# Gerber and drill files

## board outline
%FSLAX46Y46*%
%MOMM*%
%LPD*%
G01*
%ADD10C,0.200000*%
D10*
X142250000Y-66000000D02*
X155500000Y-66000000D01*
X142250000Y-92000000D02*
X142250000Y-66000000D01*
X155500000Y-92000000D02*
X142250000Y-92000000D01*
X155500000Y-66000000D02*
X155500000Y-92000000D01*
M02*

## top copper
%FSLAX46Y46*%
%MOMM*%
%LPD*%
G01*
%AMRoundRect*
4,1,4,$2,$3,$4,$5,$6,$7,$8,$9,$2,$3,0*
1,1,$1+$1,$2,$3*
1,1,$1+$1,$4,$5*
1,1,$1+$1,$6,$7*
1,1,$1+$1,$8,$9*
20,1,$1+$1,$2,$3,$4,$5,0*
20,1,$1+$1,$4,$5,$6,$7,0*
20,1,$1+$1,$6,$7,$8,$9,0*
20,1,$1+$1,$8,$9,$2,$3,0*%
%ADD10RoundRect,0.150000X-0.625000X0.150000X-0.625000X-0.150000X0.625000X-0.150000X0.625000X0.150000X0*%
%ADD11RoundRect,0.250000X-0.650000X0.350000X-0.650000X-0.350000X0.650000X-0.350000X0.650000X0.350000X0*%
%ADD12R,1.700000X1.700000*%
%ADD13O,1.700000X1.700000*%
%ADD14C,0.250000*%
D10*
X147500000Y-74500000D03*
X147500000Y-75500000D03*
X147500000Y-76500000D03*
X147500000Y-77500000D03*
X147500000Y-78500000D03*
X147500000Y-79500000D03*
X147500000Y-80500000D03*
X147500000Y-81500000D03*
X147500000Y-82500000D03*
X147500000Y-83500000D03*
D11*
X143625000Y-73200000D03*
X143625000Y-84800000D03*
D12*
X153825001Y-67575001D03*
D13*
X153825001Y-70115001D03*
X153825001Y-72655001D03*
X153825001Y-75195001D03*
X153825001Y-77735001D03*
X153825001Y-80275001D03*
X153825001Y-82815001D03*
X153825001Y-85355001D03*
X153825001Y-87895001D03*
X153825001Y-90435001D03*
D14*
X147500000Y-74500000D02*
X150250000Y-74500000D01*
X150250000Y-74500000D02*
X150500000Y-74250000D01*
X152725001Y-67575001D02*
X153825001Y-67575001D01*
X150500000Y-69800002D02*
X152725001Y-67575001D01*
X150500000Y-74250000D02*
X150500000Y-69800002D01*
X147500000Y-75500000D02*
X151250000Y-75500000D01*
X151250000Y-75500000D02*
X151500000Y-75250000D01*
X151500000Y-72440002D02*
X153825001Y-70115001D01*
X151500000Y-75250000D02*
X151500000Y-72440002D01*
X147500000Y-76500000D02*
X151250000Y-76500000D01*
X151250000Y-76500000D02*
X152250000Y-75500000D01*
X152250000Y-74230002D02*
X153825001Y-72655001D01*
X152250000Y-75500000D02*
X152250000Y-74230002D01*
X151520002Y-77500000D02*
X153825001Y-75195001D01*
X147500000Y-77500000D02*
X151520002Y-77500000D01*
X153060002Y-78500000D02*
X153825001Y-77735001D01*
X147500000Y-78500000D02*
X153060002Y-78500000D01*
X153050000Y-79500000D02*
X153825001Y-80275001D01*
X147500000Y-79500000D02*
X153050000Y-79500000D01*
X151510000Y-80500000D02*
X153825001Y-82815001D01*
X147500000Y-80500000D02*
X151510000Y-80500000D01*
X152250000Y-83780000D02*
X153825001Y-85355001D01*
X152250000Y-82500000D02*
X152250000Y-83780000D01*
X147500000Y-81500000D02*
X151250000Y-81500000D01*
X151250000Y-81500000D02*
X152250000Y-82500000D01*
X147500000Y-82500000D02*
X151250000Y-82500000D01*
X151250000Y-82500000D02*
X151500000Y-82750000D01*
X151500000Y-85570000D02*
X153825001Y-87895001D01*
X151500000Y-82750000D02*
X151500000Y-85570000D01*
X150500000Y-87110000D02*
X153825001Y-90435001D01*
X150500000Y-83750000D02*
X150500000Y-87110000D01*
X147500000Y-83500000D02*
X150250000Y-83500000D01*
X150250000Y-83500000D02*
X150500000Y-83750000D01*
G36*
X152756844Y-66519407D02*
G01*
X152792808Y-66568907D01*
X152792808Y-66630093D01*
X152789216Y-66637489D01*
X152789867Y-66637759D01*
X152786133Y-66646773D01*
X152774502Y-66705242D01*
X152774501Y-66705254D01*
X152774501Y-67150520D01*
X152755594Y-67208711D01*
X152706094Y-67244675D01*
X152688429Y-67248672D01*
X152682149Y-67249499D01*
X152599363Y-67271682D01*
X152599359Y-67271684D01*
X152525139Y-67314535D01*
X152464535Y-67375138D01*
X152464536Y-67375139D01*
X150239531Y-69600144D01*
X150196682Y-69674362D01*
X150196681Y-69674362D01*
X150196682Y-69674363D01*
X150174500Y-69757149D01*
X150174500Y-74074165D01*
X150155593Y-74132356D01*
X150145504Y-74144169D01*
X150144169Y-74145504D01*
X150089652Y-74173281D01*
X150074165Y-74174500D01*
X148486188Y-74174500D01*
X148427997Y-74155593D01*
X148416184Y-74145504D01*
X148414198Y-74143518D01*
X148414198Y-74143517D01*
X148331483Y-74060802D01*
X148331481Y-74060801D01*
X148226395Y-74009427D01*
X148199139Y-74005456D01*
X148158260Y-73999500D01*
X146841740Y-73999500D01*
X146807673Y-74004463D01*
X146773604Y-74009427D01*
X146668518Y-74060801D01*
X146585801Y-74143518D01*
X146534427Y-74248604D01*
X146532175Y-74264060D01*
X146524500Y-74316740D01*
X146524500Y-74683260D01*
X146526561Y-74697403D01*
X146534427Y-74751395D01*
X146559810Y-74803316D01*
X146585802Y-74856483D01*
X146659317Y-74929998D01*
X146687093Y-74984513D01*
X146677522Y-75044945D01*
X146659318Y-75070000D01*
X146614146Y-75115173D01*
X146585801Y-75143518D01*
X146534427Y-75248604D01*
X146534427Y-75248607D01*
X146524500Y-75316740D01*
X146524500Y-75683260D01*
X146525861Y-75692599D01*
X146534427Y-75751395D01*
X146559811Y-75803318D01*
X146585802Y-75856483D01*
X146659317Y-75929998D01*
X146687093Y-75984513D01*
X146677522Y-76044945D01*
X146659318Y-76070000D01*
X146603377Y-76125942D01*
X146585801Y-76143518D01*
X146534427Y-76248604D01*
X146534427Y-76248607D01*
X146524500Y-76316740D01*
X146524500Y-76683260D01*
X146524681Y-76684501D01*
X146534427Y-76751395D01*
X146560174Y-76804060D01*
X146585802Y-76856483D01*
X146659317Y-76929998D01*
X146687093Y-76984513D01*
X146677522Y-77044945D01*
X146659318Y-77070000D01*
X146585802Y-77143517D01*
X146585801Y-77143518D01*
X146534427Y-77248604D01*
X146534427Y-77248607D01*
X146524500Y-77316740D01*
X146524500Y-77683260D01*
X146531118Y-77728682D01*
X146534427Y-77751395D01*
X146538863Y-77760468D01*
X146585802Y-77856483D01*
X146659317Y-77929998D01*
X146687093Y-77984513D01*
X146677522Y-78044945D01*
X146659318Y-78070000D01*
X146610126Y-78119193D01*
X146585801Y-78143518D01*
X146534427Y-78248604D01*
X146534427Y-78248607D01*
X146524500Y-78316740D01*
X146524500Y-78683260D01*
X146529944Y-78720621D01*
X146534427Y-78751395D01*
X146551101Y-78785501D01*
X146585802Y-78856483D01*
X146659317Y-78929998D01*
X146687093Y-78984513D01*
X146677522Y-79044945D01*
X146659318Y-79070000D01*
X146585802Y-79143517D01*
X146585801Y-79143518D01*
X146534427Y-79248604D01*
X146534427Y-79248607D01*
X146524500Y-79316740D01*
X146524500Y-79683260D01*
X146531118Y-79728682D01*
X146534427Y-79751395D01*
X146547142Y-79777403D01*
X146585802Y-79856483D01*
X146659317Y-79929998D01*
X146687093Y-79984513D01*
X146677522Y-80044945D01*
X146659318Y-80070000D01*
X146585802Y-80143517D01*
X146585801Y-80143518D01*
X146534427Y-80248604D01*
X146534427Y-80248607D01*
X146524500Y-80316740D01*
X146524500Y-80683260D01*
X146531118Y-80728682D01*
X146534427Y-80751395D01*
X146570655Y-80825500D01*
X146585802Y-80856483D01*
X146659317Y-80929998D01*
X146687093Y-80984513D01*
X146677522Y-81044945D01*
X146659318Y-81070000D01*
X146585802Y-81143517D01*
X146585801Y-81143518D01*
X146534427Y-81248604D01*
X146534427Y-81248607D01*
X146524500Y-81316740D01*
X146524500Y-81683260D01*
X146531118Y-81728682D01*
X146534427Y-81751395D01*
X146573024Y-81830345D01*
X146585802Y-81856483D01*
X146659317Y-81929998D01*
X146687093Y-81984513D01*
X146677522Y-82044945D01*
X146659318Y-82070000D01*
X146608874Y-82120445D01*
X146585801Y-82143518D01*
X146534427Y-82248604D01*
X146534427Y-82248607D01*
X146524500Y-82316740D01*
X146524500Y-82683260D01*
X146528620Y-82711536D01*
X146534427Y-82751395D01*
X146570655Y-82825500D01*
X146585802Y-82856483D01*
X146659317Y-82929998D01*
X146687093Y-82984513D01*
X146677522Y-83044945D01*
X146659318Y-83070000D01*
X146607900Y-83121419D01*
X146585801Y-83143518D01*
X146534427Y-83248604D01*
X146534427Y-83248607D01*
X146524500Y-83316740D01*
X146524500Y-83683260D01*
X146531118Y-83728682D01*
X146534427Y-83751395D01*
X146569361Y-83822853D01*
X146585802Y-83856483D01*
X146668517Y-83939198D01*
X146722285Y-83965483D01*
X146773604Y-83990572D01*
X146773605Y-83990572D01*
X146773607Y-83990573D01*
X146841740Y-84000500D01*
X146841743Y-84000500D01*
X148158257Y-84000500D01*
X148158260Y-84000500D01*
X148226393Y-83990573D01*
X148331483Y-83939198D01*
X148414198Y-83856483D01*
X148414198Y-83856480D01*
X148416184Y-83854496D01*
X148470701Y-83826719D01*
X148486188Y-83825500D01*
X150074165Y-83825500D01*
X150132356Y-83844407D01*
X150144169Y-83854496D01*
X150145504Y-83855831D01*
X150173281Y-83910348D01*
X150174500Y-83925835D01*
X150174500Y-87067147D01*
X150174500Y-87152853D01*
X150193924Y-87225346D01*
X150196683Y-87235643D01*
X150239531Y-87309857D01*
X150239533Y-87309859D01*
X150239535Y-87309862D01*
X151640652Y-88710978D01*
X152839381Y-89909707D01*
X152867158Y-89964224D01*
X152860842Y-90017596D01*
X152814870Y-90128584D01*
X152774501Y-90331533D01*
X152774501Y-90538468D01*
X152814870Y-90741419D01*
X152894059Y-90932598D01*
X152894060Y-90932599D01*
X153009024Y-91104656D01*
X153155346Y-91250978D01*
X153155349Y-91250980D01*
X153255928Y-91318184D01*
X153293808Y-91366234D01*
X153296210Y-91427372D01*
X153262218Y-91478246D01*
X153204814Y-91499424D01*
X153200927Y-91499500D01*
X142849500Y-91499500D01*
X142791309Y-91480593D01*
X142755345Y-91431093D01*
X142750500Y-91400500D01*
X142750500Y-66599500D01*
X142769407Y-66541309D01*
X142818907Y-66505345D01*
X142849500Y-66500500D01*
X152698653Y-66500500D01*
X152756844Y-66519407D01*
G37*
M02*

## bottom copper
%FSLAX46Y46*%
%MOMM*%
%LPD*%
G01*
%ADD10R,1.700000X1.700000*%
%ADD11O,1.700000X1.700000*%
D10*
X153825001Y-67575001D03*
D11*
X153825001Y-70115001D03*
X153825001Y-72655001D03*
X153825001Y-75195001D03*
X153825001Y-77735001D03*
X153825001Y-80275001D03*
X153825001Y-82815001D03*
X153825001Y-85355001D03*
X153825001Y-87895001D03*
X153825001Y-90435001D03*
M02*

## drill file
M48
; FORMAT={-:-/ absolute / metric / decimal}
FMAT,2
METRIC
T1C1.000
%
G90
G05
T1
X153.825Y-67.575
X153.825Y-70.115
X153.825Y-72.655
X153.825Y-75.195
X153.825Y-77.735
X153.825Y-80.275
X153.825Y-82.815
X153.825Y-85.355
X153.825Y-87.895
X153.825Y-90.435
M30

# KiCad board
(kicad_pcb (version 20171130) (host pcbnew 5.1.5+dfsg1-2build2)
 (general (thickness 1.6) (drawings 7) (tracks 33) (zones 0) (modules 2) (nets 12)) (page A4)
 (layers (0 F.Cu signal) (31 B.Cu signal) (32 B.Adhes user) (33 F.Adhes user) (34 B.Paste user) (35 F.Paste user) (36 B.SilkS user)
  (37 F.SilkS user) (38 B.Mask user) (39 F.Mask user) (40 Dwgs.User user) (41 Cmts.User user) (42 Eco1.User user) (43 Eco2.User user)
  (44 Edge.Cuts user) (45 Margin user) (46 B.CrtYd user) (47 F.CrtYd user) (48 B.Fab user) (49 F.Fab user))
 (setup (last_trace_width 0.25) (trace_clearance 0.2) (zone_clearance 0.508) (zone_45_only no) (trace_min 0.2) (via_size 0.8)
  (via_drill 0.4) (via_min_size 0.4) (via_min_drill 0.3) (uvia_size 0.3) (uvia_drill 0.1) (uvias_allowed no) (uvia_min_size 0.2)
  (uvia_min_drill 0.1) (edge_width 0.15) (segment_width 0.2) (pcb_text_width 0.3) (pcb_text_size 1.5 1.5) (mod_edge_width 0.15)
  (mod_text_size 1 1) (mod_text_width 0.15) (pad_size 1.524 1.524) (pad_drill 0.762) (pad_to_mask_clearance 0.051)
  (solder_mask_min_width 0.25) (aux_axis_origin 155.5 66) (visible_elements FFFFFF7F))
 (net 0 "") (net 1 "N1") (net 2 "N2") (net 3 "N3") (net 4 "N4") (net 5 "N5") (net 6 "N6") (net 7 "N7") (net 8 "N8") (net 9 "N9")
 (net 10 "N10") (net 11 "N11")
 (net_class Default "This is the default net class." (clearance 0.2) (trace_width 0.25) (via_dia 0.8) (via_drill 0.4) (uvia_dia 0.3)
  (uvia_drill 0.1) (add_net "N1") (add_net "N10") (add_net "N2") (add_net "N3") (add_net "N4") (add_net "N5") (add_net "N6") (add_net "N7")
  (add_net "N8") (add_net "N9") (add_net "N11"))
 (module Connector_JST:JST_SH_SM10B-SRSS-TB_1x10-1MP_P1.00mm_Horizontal (layer F.Cu) (at 145.5 79 270)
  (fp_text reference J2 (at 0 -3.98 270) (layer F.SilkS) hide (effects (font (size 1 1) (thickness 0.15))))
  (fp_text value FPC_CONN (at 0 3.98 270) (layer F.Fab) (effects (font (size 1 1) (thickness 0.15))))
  (pad 1 smd roundrect (at -4.5 -2 270) (size 0.6 1.55) (layers F.Cu F.Paste F.Mask) (roundrect_rratio 0.25) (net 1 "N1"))
  (pad 2 smd roundrect (at -3.5 -2 270) (size 0.6 1.55) (layers F.Cu F.Paste F.Mask) (roundrect_rratio 0.25) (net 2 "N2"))
  (pad 3 smd roundrect (at -2.5 -2 270) (size 0.6 1.55) (layers F.Cu F.Paste F.Mask) (roundrect_rratio 0.25) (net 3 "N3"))
  (pad 4 smd roundrect (at -1.5 -2 270) (size 0.6 1.55) (layers F.Cu F.Paste F.Mask) (roundrect_rratio 0.25) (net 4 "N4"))
  (pad 5 smd roundrect (at -0.5 -2 270) (size 0.6 1.55) (layers F.Cu F.Paste F.Mask) (roundrect_rratio 0.25) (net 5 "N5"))
  (pad 6 smd roundrect (at 0.5 -2 270) (size 0.6 1.55) (layers F.Cu F.Paste F.Mask) (roundrect_rratio 0.25) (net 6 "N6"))
  (pad 7 smd roundrect (at 1.5 -2 270) (size 0.6 1.55) (layers F.Cu F.Paste F.Mask) (roundrect_rratio 0.25) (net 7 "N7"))
  (pad 8 smd roundrect (at 2.5 -2 270) (size 0.6 1.55) (layers F.Cu F.Paste F.Mask) (roundrect_rratio 0.25) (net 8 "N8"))
  (pad 9 smd roundrect (at 3.5 -2 270) (size 0.6 1.55) (layers F.Cu F.Paste F.Mask) (roundrect_rratio 0.25) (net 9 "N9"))
  (pad 10 smd roundrect (at 4.5 -2 270) (size 0.6 1.55) (layers F.Cu F.Paste F.Mask) (roundrect_rratio 0.25) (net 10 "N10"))
  (pad MP smd roundrect (at -5.8 1.875 270) (size 1.2 1.8) (layers F.Cu F.Paste F.Mask) (roundrect_rratio 0.208333) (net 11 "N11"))
  (pad MP smd roundrect (at 5.8 1.875 270) (size 1.2 1.8) (layers F.Cu F.Paste F.Mask) (roundrect_rratio 0.208333) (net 11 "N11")))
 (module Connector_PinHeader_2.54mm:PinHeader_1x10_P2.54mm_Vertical (layer F.Cu) (at 153.825001 67.575001)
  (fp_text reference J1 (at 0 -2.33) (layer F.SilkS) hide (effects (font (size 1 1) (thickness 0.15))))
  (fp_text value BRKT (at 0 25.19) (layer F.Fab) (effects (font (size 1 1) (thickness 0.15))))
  (pad 1 thru_hole rect (at 0 0) (size 1.7 1.7) (drill 1) (layers *.Cu *.Mask) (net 1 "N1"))
  (pad 2 thru_hole oval (at 0 2.54) (size 1.7 1.7) (drill 1) (layers *.Cu *.Mask) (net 2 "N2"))
  (pad 3 thru_hole oval (at 0 5.08) (size 1.7 1.7) (drill 1) (layers *.Cu *.Mask) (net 3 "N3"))
  (pad 4 thru_hole oval (at 0 7.62) (size 1.7 1.7) (drill 1) (layers *.Cu *.Mask) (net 4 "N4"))
  (pad 5 thru_hole oval (at 0 10.16) (size 1.7 1.7) (drill 1) (layers *.Cu *.Mask) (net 5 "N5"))
  (pad 6 thru_hole oval (at 0 12.7) (size 1.7 1.7) (drill 1) (layers *.Cu *.Mask) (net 6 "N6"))
  (pad 7 thru_hole oval (at 0 15.24) (size 1.7 1.7) (drill 1) (layers *.Cu *.Mask) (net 7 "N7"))
  (pad 8 thru_hole oval (at 0 17.78) (size 1.7 1.7) (drill 1) (layers *.Cu *.Mask) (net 8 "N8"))
  (pad 9 thru_hole oval (at 0 20.32) (size 1.7 1.7) (drill 1) (layers *.Cu *.Mask) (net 9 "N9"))
  (pad 10 thru_hole oval (at 0 22.86) (size 1.7 1.7) (drill 1) (layers *.Cu *.Mask) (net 10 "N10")))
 (gr_line (start 142.25 66) (end 155.5 66) (layer Edge.Cuts) (width 0.2))
 (gr_line (start 142.25 92) (end 142.25 66) (layer Edge.Cuts) (width 0.2))
 (gr_line (start 155.5 92) (end 142.25 92) (layer Edge.Cuts) (width 0.2))
 (gr_line (start 155.5 66) (end 155.5 92) (layer Edge.Cuts) (width 0.2))
 (segment (start 147.5 74.5) (end 150.25 74.5) (width 0.25) (layer F.Cu) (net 1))
 (segment (start 150.25 74.5) (end 150.5 74.25) (width 0.25) (layer F.Cu) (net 1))
 (segment (start 152.725001 67.575001) (end 153.825001 67.575001) (width 0.25) (layer F.Cu) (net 1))
 (segment (start 150.5 69.800002) (end 152.725001 67.575001) (width 0.25) (layer F.Cu) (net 1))
 (segment (start 150.5 74.25) (end 150.5 69.800002) (width 0.25) (layer F.Cu) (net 1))
 (segment (start 147.5 75.5) (end 151.25 75.5) (width 0.25) (layer F.Cu) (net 2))
 (segment (start 151.25 75.5) (end 151.5 75.25) (width 0.25) (layer F.Cu) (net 2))
 (segment (start 151.5 72.440002) (end 153.825001 70.115001) (width 0.25) (layer F.Cu) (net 2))
 (segment (start 151.5 75.25) (end 151.5 72.440002) (width 0.25) (layer F.Cu) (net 2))
 (segment (start 147.5 76.5) (end 151.25 76.5) (width 0.25) (layer F.Cu) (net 3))
 (segment (start 151.25 76.5) (end 152.25 75.5) (width 0.25) (layer F.Cu) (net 3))
 (segment (start 152.25 74.230002) (end 153.825001 72.655001) (width 0.25) (layer F.Cu) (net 3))
 (segment (start 152.25 75.5) (end 152.25 74.230002) (width 0.25) (layer F.Cu) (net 3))
 (segment (start 151.520002 77.5) (end 153.825001 75.195001) (width 0.25) (layer F.Cu) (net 4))
 (segment (start 147.5 77.5) (end 151.520002 77.5) (width 0.25) (layer F.Cu) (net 4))
 (segment (start 153.060002 78.5) (end 153.825001 77.735001) (width 0.25) (layer F.Cu) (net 5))
 (segment (start 147.5 78.5) (end 153.060002 78.5) (width 0.25) (layer F.Cu) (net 5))
 (segment (start 153.05 79.5) (end 153.825001 80.275001) (width 0.25) (layer F.Cu) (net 6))
 (segment (start 147.5 79.5) (end 153.05 79.5) (width 0.25) (layer F.Cu) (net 6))
 (segment (start 151.51 80.5) (end 153.825001 82.815001) (width 0.25) (layer F.Cu) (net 7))
 (segment (start 147.5 80.5) (end 151.51 80.5) (width 0.25) (layer F.Cu) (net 7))
 (segment (start 152.25 83.78) (end 153.825001 85.355001) (width 0.25) (layer F.Cu) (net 8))
 (segment (start 152.25 82.5) (end 152.25 83.78) (width 0.25) (layer F.Cu) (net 8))
 (segment (start 147.5 81.5) (end 151.25 81.5) (width 0.25) (layer F.Cu) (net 8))
 (segment (start 151.25 81.5) (end 152.25 82.5) (width 0.25) (layer F.Cu) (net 8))
 (segment (start 147.5 82.5) (end 151.25 82.5) (width 0.25) (layer F.Cu) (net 9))
 (segment (start 151.25 82.5) (end 151.5 82.75) (width 0.25) (layer F.Cu) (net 9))
 (segment (start 151.5 85.57) (end 153.825001 87.895001) (width 0.25) (layer F.Cu) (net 9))
 (segment (start 151.5 82.75) (end 151.5 85.57) (width 0.25) (layer F.Cu) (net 9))
 (segment (start 150.5 87.11) (end 153.825001 90.435001) (width 0.25) (layer F.Cu) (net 10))
 (segment (start 150.5 83.75) (end 150.5 87.11) (width 0.25) (layer F.Cu) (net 10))
 (segment (start 147.5 83.5) (end 150.25 83.5) (width 0.25) (layer F.Cu) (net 10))
 (segment (start 150.25 83.5) (end 150.5 83.75) (width 0.25) (layer F.Cu) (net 10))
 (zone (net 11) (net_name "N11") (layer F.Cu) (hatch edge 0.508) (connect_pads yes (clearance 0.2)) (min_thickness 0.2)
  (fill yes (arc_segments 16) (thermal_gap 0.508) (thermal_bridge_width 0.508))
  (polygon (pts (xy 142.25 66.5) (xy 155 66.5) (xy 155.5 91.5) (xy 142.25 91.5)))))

